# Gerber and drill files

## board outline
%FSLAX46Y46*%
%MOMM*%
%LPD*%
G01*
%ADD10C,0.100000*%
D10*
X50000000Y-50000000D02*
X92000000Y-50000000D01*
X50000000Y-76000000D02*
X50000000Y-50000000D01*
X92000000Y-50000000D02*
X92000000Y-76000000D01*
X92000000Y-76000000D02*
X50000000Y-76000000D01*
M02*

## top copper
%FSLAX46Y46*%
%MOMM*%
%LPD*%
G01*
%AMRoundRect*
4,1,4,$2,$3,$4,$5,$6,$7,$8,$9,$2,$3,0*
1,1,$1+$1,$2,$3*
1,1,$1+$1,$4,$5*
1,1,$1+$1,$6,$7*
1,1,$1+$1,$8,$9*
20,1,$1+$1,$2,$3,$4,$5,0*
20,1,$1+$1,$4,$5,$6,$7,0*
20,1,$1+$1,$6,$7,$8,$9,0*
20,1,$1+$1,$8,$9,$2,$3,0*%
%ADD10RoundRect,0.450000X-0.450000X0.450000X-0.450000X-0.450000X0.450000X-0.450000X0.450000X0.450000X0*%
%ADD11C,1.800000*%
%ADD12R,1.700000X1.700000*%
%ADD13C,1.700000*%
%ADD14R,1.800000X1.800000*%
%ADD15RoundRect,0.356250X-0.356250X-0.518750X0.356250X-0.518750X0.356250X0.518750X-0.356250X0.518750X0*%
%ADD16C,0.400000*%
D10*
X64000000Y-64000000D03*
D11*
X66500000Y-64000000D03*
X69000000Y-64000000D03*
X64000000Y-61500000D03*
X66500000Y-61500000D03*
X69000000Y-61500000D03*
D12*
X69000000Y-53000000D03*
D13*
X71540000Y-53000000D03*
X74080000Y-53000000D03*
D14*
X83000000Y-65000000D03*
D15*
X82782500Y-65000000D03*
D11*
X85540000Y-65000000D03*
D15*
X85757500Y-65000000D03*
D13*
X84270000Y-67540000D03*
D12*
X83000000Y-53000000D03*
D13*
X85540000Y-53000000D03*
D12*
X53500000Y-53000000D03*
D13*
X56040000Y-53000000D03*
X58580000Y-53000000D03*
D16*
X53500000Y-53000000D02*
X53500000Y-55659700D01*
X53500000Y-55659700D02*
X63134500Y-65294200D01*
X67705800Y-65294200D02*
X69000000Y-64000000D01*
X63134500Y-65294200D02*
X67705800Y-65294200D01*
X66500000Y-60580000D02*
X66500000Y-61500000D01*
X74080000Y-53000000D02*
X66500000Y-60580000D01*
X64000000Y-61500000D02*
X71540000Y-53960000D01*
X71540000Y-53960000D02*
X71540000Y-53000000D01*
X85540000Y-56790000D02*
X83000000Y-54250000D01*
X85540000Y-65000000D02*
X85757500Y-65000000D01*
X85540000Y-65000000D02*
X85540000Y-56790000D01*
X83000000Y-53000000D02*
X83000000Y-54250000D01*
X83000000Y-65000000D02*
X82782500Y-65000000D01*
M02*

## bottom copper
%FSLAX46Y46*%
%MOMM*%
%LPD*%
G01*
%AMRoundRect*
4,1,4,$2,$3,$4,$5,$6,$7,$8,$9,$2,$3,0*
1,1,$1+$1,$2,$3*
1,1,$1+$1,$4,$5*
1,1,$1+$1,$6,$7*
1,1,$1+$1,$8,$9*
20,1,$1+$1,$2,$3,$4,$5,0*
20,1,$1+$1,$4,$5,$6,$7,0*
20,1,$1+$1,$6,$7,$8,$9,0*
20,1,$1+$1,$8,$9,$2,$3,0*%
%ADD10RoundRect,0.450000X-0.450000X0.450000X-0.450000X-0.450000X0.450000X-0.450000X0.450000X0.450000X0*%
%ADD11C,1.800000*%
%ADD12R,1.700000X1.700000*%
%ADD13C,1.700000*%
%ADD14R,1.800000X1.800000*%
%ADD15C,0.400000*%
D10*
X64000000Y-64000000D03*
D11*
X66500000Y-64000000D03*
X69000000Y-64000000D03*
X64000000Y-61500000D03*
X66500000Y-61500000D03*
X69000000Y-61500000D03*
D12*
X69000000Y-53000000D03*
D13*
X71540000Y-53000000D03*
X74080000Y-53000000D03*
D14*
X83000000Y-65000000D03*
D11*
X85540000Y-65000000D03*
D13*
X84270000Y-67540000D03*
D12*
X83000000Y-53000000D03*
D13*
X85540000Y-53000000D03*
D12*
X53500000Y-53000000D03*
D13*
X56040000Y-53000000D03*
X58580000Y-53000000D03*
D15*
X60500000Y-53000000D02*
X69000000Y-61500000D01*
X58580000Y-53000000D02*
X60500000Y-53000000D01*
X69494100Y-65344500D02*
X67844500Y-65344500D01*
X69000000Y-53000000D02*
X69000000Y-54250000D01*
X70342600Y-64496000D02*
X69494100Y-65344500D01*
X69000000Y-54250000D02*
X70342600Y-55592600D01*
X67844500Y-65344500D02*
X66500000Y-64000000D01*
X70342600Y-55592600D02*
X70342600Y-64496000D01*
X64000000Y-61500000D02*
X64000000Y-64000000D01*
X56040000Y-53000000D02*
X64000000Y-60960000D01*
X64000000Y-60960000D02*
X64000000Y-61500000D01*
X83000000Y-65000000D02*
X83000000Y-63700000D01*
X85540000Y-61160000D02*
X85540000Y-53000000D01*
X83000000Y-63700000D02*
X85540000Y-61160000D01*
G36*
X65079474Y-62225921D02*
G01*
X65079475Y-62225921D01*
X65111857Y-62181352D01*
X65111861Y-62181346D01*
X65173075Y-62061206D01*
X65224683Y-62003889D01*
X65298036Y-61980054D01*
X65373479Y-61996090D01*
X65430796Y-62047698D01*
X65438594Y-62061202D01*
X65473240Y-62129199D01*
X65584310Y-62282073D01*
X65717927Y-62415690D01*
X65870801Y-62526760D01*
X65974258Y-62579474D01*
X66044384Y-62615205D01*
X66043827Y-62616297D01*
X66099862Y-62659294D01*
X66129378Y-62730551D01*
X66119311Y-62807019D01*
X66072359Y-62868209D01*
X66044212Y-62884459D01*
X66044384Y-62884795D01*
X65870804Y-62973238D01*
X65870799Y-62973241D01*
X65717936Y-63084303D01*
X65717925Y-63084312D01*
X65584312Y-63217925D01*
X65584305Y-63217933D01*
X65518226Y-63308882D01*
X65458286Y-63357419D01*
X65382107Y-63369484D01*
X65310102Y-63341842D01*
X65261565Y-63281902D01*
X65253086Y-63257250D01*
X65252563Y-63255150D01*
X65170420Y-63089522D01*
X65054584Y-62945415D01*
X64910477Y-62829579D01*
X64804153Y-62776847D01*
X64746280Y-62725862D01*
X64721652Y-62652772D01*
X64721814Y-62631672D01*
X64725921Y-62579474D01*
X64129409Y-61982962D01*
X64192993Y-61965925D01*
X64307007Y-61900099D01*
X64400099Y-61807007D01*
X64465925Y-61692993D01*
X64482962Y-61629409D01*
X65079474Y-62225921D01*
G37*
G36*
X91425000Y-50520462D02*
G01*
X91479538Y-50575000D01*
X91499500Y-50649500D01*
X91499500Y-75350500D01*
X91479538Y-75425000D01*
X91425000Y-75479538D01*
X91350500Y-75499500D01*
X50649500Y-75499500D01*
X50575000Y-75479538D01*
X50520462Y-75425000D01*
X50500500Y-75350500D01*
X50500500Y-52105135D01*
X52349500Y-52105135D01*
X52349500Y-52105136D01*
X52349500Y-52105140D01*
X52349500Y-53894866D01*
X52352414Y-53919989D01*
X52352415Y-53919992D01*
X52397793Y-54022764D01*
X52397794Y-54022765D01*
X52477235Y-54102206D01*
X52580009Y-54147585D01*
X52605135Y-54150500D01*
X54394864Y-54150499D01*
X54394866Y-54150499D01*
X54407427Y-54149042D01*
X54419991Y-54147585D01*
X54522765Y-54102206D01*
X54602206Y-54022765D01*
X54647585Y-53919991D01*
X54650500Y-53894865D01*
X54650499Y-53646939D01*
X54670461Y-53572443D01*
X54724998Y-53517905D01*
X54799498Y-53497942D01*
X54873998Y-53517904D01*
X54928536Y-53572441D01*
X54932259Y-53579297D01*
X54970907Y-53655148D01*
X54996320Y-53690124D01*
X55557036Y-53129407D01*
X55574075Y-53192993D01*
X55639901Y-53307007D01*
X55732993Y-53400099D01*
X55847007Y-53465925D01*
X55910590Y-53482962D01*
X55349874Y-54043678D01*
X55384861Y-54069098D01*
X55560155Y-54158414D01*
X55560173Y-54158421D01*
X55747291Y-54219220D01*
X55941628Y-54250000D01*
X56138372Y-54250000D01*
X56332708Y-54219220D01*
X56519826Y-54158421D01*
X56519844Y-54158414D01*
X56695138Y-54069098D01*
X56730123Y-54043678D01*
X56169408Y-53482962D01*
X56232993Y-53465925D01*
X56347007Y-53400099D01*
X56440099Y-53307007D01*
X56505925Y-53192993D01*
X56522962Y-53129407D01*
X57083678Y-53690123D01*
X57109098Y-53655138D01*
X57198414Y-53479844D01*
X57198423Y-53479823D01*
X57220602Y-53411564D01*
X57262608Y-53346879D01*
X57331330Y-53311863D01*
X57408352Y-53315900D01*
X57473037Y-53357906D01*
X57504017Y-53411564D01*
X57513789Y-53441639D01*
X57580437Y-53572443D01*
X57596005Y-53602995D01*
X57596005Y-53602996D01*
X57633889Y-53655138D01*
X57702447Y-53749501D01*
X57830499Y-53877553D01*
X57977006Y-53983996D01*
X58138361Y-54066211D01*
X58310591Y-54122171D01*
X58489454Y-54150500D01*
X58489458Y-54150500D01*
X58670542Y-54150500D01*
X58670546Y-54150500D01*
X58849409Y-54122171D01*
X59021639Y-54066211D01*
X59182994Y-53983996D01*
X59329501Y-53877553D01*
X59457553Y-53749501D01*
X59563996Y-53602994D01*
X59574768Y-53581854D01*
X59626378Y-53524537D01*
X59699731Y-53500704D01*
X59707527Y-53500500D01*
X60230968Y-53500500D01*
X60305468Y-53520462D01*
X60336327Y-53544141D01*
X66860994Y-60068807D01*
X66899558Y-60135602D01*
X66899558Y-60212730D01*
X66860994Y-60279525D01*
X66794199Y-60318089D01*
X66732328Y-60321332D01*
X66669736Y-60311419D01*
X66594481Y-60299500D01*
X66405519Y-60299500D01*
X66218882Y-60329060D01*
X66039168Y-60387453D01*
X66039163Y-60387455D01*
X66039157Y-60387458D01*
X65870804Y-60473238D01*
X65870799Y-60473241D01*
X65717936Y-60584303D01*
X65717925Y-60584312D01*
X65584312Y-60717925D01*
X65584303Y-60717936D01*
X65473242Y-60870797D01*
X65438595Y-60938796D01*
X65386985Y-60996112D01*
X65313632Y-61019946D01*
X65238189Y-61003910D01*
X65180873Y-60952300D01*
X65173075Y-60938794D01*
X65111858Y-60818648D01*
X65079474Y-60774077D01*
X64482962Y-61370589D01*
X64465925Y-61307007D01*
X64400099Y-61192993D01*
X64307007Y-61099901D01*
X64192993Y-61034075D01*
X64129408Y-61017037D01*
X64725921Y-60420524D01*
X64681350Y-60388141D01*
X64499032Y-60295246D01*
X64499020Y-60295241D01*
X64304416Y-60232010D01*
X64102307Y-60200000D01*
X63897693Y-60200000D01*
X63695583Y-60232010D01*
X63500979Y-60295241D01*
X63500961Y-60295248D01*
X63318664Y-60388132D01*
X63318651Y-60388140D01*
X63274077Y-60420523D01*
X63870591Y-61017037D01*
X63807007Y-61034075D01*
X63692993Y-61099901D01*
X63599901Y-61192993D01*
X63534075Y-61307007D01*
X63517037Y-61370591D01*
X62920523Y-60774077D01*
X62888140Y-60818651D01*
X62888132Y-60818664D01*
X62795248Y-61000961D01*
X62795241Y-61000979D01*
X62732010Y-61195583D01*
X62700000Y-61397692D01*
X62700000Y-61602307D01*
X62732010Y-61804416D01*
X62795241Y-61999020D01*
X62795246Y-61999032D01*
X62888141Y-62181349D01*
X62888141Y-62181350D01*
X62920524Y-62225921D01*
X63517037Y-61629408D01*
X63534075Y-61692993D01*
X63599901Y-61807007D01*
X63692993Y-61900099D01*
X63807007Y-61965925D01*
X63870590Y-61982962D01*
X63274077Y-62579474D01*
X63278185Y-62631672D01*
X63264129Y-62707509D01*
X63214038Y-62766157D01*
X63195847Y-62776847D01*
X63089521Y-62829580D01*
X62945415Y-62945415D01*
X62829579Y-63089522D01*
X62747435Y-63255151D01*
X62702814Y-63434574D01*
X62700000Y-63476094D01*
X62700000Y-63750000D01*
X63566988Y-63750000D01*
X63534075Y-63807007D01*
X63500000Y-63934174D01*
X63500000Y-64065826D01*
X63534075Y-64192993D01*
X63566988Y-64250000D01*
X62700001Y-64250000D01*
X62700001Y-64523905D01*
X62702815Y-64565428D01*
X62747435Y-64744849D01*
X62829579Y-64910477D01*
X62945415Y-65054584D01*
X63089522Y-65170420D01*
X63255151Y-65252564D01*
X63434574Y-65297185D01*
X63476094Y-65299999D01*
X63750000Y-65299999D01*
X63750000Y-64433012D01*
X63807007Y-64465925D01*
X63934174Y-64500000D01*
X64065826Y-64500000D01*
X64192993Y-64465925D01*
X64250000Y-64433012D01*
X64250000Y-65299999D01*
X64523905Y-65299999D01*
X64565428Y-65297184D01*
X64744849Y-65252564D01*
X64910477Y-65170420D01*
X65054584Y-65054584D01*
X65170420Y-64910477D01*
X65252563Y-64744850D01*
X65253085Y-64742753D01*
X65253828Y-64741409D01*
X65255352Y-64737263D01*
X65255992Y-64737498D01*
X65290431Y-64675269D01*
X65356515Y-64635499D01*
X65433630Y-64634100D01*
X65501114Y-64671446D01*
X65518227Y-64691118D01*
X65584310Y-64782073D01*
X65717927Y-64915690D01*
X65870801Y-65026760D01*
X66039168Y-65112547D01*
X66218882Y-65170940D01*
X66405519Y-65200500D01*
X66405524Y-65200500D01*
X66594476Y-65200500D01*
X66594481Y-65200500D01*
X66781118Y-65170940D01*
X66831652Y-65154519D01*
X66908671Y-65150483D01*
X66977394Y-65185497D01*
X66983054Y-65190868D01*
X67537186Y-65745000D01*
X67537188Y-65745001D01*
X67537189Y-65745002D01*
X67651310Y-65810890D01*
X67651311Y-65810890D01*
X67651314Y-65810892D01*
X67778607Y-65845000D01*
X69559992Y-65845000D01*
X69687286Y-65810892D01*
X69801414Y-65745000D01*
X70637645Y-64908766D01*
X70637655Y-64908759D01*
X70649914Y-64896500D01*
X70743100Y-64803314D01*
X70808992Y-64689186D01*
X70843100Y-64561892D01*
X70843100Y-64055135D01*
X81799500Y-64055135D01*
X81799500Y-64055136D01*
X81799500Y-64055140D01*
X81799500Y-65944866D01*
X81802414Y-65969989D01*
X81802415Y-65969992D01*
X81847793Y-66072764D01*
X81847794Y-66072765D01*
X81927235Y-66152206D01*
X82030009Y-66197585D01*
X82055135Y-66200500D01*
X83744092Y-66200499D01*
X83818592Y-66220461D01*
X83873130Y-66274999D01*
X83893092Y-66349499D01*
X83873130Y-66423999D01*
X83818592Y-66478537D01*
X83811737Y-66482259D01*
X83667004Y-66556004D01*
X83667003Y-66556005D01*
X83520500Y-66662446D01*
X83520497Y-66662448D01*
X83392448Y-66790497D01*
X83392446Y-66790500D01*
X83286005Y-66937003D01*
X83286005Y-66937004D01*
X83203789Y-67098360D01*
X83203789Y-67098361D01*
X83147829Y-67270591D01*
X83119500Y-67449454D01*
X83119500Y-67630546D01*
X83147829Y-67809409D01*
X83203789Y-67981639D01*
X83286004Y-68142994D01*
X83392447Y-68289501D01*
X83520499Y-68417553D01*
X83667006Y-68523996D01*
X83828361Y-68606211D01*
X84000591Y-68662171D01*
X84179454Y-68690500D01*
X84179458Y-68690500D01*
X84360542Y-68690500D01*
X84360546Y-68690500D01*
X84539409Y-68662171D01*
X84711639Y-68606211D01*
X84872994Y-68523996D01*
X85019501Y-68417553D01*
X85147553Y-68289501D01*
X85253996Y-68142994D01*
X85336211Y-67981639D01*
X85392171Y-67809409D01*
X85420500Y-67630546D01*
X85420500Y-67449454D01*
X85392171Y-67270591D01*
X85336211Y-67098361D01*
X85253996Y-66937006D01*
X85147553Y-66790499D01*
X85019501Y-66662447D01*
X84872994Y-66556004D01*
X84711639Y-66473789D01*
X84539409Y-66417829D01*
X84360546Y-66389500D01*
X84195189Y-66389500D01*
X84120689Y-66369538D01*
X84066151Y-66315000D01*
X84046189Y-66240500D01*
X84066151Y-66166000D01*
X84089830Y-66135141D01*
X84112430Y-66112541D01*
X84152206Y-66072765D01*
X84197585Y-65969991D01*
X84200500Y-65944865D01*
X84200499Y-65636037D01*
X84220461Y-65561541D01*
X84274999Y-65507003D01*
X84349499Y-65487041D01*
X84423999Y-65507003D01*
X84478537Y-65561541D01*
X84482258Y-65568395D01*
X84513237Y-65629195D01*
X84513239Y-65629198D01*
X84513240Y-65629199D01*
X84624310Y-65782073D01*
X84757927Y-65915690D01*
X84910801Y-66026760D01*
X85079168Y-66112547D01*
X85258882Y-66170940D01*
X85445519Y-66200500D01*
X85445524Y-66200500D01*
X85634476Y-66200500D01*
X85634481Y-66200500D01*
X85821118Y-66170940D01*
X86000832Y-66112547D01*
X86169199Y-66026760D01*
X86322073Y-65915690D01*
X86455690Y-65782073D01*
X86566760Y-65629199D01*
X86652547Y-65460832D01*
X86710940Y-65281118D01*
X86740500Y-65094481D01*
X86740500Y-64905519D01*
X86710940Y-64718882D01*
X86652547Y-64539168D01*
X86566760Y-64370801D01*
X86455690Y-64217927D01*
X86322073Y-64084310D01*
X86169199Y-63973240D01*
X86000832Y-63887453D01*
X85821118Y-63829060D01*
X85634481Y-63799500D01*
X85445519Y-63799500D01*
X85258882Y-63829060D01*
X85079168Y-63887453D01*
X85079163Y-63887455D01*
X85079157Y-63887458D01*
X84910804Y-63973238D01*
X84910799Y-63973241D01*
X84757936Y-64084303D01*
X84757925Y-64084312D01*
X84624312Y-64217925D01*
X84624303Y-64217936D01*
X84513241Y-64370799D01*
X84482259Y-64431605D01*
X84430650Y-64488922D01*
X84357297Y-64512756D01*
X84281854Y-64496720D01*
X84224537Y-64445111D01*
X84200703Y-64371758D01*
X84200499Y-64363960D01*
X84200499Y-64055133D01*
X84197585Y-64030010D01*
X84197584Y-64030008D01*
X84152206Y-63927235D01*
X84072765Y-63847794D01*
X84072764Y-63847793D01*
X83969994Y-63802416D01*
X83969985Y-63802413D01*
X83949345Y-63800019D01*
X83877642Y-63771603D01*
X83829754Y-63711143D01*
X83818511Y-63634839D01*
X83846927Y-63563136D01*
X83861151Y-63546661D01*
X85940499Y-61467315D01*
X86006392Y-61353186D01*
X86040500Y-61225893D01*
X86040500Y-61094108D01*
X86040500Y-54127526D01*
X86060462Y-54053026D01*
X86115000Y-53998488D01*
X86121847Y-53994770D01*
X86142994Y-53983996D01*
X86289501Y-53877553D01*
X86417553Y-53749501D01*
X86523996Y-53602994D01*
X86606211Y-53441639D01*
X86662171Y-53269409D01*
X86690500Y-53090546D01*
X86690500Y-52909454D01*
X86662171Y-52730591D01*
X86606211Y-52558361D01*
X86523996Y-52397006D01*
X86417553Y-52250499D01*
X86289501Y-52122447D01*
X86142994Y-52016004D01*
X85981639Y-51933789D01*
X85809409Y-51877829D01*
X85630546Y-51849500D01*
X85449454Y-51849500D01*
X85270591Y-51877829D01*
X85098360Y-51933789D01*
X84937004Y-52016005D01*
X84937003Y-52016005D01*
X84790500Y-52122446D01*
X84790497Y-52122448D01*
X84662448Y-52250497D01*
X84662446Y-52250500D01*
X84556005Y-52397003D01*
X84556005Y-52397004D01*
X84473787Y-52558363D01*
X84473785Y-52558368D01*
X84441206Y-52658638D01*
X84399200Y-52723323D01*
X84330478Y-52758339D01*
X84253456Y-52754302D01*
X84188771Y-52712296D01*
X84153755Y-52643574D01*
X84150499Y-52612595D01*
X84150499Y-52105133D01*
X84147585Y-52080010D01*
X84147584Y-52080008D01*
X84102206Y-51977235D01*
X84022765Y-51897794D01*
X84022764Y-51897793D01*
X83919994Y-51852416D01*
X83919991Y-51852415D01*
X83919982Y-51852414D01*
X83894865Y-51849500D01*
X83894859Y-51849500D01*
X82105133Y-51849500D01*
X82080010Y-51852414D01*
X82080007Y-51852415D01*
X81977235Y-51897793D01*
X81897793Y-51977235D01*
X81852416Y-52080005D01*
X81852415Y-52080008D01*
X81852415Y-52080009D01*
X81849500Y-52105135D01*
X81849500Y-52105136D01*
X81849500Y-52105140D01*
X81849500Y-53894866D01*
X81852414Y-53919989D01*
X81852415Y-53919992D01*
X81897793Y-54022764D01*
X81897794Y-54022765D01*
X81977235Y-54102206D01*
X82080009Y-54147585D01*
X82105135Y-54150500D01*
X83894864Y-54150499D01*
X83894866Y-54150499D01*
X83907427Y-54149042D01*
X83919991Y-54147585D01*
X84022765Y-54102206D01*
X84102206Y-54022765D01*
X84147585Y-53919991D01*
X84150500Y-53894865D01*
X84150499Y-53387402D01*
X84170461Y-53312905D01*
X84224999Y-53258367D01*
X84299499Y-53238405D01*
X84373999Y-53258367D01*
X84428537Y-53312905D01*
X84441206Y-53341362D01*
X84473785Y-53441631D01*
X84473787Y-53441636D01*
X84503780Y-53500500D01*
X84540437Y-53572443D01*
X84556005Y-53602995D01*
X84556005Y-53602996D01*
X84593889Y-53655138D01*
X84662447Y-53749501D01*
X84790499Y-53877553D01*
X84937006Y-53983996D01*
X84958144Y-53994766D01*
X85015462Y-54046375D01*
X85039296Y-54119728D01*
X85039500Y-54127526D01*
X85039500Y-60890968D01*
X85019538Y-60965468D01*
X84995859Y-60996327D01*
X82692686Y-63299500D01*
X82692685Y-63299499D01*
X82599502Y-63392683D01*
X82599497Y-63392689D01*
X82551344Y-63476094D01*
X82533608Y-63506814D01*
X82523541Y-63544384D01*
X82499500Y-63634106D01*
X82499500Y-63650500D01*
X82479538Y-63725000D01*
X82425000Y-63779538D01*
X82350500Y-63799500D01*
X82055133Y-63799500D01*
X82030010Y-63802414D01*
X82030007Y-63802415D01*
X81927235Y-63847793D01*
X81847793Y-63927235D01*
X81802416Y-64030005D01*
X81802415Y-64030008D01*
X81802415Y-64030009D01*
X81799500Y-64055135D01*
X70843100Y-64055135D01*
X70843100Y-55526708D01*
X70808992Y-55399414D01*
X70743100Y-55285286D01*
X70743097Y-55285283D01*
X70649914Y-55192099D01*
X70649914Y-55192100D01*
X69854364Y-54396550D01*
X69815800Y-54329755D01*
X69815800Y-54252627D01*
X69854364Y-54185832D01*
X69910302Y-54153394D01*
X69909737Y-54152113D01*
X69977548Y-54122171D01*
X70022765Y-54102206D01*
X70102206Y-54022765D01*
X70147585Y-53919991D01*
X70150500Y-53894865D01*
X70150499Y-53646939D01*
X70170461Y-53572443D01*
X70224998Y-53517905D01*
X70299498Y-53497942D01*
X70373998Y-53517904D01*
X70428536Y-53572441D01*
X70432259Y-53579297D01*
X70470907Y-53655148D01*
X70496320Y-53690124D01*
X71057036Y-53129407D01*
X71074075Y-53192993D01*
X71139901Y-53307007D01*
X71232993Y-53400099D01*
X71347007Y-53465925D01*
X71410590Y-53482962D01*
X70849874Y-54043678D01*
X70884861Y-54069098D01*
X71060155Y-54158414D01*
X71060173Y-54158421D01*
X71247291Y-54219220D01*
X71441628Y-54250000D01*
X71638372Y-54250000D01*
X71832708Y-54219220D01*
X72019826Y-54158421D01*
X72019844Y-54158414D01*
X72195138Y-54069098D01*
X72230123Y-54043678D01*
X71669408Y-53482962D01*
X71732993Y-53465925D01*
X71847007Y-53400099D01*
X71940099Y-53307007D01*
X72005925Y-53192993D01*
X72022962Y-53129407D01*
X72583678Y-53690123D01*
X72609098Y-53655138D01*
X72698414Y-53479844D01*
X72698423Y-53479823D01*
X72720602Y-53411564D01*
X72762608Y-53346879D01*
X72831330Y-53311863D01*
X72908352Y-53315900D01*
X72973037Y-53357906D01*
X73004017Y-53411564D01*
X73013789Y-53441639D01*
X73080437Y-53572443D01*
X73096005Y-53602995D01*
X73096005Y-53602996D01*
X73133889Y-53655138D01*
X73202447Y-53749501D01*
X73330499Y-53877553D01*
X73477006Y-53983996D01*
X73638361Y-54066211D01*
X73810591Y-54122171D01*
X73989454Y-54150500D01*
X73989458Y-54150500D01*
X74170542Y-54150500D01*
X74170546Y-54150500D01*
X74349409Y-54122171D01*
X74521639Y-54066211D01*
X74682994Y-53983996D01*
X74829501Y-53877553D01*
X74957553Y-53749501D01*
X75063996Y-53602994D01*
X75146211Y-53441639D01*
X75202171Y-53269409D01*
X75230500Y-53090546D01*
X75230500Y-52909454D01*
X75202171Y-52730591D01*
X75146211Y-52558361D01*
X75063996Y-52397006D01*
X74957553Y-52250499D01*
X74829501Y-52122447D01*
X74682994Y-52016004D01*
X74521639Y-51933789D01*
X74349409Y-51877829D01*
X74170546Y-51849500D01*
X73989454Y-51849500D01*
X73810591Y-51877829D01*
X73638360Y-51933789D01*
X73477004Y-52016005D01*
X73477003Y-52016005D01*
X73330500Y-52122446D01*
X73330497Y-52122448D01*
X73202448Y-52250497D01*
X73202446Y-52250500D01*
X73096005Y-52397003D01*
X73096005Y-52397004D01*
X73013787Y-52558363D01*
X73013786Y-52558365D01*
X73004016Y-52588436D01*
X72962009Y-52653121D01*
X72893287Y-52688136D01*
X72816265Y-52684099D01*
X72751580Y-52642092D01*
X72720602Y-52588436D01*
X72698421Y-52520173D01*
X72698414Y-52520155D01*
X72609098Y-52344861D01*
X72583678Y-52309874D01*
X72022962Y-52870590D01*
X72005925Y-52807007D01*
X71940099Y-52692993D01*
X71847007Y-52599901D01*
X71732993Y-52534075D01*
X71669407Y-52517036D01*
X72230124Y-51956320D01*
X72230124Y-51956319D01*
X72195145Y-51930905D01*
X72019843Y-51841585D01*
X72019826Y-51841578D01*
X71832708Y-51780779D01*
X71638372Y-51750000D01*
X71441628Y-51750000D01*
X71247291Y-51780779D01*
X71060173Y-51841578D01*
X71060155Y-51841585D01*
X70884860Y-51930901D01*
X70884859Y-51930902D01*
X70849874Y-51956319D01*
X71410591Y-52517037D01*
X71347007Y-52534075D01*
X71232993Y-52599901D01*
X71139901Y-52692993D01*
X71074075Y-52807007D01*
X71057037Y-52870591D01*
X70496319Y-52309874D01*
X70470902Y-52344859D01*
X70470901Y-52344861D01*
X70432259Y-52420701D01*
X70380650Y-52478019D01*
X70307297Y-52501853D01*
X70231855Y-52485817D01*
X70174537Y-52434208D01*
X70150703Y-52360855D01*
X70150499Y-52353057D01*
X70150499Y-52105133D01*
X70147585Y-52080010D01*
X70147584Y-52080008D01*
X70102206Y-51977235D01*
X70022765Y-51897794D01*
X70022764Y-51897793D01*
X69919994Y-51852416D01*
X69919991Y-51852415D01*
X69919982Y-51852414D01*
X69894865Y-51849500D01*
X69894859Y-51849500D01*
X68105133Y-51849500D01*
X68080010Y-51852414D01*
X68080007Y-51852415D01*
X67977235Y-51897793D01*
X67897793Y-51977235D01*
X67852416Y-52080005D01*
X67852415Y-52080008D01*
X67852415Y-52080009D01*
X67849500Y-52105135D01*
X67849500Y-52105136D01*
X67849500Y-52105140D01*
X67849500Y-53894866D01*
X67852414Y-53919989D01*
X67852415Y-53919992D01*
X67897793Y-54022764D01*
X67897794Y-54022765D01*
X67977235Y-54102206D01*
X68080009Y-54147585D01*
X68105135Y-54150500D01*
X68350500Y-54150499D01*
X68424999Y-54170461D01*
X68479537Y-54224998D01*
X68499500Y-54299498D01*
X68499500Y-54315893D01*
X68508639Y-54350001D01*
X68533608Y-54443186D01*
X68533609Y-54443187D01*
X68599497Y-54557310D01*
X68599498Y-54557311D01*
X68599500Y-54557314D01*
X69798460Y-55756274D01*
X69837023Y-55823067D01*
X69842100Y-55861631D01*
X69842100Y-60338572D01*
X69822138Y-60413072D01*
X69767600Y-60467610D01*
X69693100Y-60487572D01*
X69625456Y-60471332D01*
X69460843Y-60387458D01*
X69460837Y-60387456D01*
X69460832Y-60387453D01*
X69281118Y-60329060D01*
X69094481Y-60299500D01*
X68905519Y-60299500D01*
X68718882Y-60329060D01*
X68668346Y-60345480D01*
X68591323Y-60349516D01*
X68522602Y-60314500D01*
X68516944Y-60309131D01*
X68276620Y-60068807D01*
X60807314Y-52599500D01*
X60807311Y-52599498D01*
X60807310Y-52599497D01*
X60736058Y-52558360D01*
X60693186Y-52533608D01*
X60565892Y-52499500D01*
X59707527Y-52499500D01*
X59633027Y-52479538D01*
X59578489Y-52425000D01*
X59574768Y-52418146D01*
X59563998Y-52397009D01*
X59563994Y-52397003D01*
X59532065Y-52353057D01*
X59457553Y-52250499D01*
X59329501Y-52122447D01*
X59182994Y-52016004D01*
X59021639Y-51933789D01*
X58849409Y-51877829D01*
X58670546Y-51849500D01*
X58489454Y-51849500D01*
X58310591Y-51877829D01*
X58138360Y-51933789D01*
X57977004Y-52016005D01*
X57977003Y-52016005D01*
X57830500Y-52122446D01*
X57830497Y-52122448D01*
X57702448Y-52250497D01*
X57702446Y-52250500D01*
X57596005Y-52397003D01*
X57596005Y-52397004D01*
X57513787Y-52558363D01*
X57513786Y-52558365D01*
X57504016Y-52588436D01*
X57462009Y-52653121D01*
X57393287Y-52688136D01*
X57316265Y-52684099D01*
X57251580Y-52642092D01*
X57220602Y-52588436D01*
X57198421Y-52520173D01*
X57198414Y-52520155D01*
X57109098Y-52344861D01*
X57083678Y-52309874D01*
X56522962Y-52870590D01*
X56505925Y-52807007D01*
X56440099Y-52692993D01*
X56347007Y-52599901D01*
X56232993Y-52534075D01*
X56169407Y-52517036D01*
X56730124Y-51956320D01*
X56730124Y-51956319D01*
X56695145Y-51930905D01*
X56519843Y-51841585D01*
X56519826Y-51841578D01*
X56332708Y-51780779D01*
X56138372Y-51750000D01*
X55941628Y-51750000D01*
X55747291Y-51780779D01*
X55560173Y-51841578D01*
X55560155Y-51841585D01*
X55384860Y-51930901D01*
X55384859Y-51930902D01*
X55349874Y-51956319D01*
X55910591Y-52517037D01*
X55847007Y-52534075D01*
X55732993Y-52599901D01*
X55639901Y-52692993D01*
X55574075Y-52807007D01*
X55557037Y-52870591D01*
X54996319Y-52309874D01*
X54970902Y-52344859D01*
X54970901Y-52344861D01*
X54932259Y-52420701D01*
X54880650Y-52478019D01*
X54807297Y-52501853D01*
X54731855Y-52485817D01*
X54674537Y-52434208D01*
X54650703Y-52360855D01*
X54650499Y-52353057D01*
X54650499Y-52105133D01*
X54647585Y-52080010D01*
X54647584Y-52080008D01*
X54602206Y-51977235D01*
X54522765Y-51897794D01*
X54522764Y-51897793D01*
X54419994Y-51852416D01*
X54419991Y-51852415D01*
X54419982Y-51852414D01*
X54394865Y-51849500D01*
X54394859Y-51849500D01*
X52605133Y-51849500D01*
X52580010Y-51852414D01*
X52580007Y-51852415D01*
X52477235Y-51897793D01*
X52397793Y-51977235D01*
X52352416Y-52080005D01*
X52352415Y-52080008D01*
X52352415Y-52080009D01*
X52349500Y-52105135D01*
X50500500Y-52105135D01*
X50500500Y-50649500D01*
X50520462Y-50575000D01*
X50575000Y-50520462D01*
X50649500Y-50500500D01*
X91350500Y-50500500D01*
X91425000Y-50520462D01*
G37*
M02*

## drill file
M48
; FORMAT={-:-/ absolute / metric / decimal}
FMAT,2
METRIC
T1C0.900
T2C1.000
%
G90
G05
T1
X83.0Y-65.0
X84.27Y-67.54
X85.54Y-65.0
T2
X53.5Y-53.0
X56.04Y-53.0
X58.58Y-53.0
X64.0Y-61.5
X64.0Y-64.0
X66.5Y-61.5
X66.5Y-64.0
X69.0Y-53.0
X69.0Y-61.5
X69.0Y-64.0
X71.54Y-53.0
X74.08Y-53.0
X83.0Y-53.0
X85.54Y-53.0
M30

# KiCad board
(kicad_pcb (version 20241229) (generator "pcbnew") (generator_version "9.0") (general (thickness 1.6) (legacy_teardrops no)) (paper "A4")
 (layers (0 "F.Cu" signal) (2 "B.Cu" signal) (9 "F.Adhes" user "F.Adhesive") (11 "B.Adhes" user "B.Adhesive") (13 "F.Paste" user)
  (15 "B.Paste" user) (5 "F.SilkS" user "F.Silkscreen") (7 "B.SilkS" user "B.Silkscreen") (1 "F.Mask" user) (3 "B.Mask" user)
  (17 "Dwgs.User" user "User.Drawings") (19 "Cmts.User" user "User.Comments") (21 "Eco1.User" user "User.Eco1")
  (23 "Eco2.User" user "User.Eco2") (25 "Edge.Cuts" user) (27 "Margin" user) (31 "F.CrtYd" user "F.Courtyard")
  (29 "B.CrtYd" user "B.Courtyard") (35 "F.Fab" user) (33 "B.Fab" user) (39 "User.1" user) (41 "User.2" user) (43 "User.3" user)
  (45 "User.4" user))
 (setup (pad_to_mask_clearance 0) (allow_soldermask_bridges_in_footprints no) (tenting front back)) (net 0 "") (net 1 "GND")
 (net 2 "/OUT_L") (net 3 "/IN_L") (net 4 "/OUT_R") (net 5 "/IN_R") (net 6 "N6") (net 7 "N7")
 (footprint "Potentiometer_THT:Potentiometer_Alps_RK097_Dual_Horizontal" (layer "F.Cu") (at 64 64 90)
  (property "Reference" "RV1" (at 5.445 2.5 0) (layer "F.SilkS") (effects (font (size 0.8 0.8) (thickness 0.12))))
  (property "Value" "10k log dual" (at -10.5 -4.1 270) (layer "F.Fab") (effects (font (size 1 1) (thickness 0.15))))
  (pad "1" thru_hole roundrect (at 0 0 270) (size 1.8 1.8) (drill 1) (layers "*.Cu" "*.Mask") (remove_unused_layers no)
   (roundrect_rratio 0.25) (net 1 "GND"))
  (pad "2" thru_hole circle (at 0 2.5 270) (size 1.8 1.8) (drill 1) (layers "*.Cu" "*.Mask") (remove_unused_layers no) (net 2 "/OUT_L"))
  (pad "3" thru_hole circle (at 0 5 270) (size 1.8 1.8) (drill 1) (layers "*.Cu" "*.Mask") (remove_unused_layers no) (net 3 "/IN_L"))
  (pad "4" thru_hole circle (at 2.5 0 270) (size 1.8 1.8) (drill 1) (layers "*.Cu" "*.Mask") (remove_unused_layers no) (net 1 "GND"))
  (pad "5" thru_hole circle (at 2.5 2.5 270) (size 1.8 1.8) (drill 1) (layers "*.Cu" "*.Mask") (remove_unused_layers no) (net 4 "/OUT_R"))
  (pad "6" thru_hole circle (at 2.5 5 270) (size 1.8 1.8) (drill 1) (layers "*.Cu" "*.Mask") (remove_unused_layers no) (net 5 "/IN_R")))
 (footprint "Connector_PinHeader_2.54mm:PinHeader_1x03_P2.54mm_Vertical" (layer "F.Cu") (at 69 53 90)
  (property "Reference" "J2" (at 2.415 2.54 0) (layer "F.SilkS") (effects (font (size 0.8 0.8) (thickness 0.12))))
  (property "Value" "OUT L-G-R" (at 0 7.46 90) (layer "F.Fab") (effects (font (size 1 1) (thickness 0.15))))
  (pad "1" thru_hole rect (at 0 0 90) (size 1.7 1.7) (drill 1) (layers "*.Cu" "*.Mask") (remove_unused_layers no) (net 2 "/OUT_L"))
  (pad "2" thru_hole circle (at 0 2.54 90) (size 1.7 1.7) (drill 1) (layers "*.Cu" "*.Mask") (remove_unused_layers no) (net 1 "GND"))
  (pad "3" thru_hole circle (at 0 5.08 90) (size 1.7 1.7) (drill 1) (layers "*.Cu" "*.Mask") (remove_unused_layers no) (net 4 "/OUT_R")))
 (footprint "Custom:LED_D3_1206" (layer "F.Cu") (at 83 65)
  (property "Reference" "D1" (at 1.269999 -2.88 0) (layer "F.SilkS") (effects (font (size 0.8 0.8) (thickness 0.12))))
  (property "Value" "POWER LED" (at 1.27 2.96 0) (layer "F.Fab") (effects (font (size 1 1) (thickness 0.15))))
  (pad "1" thru_hole rect (at 0 0) (size 1.8 1.8) (drill 0.9) (layers "*.Cu" "*.Mask") (remove_unused_layers no) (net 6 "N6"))
  (pad "1S" smd roundrect (at -0.2175 0) (size 1.425 1.75) (layers "F.Cu" "F.Mask" "F.Paste") (roundrect_rratio 0.25) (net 6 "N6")
   (zone_connect 2) (thermal_bridge_angle 45))
  (pad "2" thru_hole circle (at 2.54 0) (size 1.8 1.8) (drill 0.9) (layers "*.Cu" "*.Mask") (remove_unused_layers no) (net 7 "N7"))
  (pad "2S" smd roundrect (at 2.7575 0) (size 1.425 1.75) (layers "F.Cu" "F.Mask" "F.Paste") (roundrect_rratio 0.25) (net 7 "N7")
   (zone_connect 2) (thermal_bridge_angle 45))
  (pad "M" thru_hole circle (at 1.27 2.54) (size 1.7 1.7) (drill 0.9) (layers "*.Cu" "*.Mask") (remove_unused_layers no)))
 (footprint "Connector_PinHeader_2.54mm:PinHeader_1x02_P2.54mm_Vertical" (layer "F.Cu") (at 83 53 90)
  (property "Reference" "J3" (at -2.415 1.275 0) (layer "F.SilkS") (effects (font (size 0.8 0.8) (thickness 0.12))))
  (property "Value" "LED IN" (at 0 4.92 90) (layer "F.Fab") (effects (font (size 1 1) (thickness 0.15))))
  (pad "1" thru_hole rect (at 0 0 90) (size 1.7 1.7) (drill 1) (layers "*.Cu" "*.Mask") (remove_unused_layers no) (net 7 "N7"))
  (pad "2" thru_hole circle (at 0 2.54 90) (size 1.7 1.7) (drill 1) (layers "*.Cu" "*.Mask") (remove_unused_layers no) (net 6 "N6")))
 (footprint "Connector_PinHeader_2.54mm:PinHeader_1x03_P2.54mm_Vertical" (layer "F.Cu") (at 53.5 53 90)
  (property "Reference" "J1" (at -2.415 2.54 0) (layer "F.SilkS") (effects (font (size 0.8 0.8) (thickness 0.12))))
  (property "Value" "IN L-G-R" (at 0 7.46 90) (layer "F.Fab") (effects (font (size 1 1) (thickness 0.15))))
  (pad "1" thru_hole rect (at 0 0 90) (size 1.7 1.7) (drill 1) (layers "*.Cu" "*.Mask") (remove_unused_layers no) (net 3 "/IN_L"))
  (pad "2" thru_hole circle (at 0 2.54 90) (size 1.7 1.7) (drill 1) (layers "*.Cu" "*.Mask") (remove_unused_layers no) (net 1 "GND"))
  (pad "3" thru_hole circle (at 0 5.08 90) (size 1.7 1.7) (drill 1) (layers "*.Cu" "*.Mask") (remove_unused_layers no) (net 5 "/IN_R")))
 (gr_line (start 50 50) (end 92 50) (stroke (width 0.1) (type default)) (layer "Edge.Cuts"))
 (gr_line (start 50 76) (end 50 50) (stroke (width 0.1) (type default)) (layer "Edge.Cuts"))
 (gr_line (start 92 50) (end 92 76) (stroke (width 0.1) (type default)) (layer "Edge.Cuts"))
 (gr_line (start 92 76) (end 50 76) (stroke (width 0.1) (type default)) (layer "Edge.Cuts"))
 (segment (start 53.5 53) (end 53.5 55.6597) (width 0.4) (layer "F.Cu") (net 3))
 (segment (start 53.5 55.6597) (end 63.1345 65.2942) (width 0.4) (layer "F.Cu") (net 3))
 (segment (start 67.7058 65.2942) (end 69 64) (width 0.4) (layer "F.Cu") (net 3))
 (segment (start 63.1345 65.2942) (end 67.7058 65.2942) (width 0.4) (layer "F.Cu") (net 3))
 (segment (start 60.5 53) (end 69 61.5) (width 0.4) (layer "B.Cu") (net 5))
 (segment (start 58.58 53) (end 60.5 53) (width 0.4) (layer "B.Cu") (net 5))
 (segment (start 69.4941 65.3445) (end 67.8445 65.3445) (width 0.4) (layer "B.Cu") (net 2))
 (segment (start 69 53) (end 69 54.25) (width 0.4) (layer "B.Cu") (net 2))
 (segment (start 70.3426 64.496) (end 69.4941 65.3445) (width 0.4) (layer "B.Cu") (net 2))
 (segment (start 69 54.25) (end 70.3426 55.5926) (width 0.4) (layer "B.Cu") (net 2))
 (segment (start 67.8445 65.3445) (end 66.5 64) (width 0.4) (layer "B.Cu") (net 2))
 (segment (start 70.3426 55.5926) (end 70.3426 64.496) (width 0.4) (layer "B.Cu") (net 2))
 (segment (start 66.5 60.58) (end 66.5 61.5) (width 0.4) (layer "F.Cu") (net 4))
 (segment (start 74.08 53) (end 66.5 60.58) (width 0.4) (layer "F.Cu") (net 4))
 (segment (start 64 61.5) (end 71.54 53.96) (width 0.4) (layer "F.Cu") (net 1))
 (segment (start 71.54 53.96) (end 71.54 53) (width 0.4) (layer "F.Cu") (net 1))
 (segment (start 64 61.5) (end 64 64) (width 0.4) (layer "B.Cu") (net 1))
 (segment (start 56.04 53) (end 64 60.96) (width 0.4) (layer "B.Cu") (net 1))
 (segment (start 64 60.96) (end 64 61.5) (width 0.4) (layer "B.Cu") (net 1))
 (segment (start 85.54 56.79) (end 83 54.25) (width 0.4) (layer "F.Cu") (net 7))
 (segment (start 85.54 65) (end 85.7575 65) (width 0.4) (layer "F.Cu") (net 7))
 (segment (start 85.54 65) (end 85.54 56.79) (width 0.4) (layer "F.Cu") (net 7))
 (segment (start 83 53) (end 83 54.25) (width 0.4) (layer "F.Cu") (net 7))
 (segment (start 83 65) (end 82.7825 65) (width 0.4) (layer "F.Cu") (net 6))
 (segment (start 83 65) (end 83 63.7) (width 0.4) (layer "B.Cu") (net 6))
 (segment (start 85.54 61.16) (end 85.54 53) (width 0.4) (layer "B.Cu") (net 6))
 (segment (start 83 63.7) (end 85.54 61.16) (width 0.4) (layer "B.Cu") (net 6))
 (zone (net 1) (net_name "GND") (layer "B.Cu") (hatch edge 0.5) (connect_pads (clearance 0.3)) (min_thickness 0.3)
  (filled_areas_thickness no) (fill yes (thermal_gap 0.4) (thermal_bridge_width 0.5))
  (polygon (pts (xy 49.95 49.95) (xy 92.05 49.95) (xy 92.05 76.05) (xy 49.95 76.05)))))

